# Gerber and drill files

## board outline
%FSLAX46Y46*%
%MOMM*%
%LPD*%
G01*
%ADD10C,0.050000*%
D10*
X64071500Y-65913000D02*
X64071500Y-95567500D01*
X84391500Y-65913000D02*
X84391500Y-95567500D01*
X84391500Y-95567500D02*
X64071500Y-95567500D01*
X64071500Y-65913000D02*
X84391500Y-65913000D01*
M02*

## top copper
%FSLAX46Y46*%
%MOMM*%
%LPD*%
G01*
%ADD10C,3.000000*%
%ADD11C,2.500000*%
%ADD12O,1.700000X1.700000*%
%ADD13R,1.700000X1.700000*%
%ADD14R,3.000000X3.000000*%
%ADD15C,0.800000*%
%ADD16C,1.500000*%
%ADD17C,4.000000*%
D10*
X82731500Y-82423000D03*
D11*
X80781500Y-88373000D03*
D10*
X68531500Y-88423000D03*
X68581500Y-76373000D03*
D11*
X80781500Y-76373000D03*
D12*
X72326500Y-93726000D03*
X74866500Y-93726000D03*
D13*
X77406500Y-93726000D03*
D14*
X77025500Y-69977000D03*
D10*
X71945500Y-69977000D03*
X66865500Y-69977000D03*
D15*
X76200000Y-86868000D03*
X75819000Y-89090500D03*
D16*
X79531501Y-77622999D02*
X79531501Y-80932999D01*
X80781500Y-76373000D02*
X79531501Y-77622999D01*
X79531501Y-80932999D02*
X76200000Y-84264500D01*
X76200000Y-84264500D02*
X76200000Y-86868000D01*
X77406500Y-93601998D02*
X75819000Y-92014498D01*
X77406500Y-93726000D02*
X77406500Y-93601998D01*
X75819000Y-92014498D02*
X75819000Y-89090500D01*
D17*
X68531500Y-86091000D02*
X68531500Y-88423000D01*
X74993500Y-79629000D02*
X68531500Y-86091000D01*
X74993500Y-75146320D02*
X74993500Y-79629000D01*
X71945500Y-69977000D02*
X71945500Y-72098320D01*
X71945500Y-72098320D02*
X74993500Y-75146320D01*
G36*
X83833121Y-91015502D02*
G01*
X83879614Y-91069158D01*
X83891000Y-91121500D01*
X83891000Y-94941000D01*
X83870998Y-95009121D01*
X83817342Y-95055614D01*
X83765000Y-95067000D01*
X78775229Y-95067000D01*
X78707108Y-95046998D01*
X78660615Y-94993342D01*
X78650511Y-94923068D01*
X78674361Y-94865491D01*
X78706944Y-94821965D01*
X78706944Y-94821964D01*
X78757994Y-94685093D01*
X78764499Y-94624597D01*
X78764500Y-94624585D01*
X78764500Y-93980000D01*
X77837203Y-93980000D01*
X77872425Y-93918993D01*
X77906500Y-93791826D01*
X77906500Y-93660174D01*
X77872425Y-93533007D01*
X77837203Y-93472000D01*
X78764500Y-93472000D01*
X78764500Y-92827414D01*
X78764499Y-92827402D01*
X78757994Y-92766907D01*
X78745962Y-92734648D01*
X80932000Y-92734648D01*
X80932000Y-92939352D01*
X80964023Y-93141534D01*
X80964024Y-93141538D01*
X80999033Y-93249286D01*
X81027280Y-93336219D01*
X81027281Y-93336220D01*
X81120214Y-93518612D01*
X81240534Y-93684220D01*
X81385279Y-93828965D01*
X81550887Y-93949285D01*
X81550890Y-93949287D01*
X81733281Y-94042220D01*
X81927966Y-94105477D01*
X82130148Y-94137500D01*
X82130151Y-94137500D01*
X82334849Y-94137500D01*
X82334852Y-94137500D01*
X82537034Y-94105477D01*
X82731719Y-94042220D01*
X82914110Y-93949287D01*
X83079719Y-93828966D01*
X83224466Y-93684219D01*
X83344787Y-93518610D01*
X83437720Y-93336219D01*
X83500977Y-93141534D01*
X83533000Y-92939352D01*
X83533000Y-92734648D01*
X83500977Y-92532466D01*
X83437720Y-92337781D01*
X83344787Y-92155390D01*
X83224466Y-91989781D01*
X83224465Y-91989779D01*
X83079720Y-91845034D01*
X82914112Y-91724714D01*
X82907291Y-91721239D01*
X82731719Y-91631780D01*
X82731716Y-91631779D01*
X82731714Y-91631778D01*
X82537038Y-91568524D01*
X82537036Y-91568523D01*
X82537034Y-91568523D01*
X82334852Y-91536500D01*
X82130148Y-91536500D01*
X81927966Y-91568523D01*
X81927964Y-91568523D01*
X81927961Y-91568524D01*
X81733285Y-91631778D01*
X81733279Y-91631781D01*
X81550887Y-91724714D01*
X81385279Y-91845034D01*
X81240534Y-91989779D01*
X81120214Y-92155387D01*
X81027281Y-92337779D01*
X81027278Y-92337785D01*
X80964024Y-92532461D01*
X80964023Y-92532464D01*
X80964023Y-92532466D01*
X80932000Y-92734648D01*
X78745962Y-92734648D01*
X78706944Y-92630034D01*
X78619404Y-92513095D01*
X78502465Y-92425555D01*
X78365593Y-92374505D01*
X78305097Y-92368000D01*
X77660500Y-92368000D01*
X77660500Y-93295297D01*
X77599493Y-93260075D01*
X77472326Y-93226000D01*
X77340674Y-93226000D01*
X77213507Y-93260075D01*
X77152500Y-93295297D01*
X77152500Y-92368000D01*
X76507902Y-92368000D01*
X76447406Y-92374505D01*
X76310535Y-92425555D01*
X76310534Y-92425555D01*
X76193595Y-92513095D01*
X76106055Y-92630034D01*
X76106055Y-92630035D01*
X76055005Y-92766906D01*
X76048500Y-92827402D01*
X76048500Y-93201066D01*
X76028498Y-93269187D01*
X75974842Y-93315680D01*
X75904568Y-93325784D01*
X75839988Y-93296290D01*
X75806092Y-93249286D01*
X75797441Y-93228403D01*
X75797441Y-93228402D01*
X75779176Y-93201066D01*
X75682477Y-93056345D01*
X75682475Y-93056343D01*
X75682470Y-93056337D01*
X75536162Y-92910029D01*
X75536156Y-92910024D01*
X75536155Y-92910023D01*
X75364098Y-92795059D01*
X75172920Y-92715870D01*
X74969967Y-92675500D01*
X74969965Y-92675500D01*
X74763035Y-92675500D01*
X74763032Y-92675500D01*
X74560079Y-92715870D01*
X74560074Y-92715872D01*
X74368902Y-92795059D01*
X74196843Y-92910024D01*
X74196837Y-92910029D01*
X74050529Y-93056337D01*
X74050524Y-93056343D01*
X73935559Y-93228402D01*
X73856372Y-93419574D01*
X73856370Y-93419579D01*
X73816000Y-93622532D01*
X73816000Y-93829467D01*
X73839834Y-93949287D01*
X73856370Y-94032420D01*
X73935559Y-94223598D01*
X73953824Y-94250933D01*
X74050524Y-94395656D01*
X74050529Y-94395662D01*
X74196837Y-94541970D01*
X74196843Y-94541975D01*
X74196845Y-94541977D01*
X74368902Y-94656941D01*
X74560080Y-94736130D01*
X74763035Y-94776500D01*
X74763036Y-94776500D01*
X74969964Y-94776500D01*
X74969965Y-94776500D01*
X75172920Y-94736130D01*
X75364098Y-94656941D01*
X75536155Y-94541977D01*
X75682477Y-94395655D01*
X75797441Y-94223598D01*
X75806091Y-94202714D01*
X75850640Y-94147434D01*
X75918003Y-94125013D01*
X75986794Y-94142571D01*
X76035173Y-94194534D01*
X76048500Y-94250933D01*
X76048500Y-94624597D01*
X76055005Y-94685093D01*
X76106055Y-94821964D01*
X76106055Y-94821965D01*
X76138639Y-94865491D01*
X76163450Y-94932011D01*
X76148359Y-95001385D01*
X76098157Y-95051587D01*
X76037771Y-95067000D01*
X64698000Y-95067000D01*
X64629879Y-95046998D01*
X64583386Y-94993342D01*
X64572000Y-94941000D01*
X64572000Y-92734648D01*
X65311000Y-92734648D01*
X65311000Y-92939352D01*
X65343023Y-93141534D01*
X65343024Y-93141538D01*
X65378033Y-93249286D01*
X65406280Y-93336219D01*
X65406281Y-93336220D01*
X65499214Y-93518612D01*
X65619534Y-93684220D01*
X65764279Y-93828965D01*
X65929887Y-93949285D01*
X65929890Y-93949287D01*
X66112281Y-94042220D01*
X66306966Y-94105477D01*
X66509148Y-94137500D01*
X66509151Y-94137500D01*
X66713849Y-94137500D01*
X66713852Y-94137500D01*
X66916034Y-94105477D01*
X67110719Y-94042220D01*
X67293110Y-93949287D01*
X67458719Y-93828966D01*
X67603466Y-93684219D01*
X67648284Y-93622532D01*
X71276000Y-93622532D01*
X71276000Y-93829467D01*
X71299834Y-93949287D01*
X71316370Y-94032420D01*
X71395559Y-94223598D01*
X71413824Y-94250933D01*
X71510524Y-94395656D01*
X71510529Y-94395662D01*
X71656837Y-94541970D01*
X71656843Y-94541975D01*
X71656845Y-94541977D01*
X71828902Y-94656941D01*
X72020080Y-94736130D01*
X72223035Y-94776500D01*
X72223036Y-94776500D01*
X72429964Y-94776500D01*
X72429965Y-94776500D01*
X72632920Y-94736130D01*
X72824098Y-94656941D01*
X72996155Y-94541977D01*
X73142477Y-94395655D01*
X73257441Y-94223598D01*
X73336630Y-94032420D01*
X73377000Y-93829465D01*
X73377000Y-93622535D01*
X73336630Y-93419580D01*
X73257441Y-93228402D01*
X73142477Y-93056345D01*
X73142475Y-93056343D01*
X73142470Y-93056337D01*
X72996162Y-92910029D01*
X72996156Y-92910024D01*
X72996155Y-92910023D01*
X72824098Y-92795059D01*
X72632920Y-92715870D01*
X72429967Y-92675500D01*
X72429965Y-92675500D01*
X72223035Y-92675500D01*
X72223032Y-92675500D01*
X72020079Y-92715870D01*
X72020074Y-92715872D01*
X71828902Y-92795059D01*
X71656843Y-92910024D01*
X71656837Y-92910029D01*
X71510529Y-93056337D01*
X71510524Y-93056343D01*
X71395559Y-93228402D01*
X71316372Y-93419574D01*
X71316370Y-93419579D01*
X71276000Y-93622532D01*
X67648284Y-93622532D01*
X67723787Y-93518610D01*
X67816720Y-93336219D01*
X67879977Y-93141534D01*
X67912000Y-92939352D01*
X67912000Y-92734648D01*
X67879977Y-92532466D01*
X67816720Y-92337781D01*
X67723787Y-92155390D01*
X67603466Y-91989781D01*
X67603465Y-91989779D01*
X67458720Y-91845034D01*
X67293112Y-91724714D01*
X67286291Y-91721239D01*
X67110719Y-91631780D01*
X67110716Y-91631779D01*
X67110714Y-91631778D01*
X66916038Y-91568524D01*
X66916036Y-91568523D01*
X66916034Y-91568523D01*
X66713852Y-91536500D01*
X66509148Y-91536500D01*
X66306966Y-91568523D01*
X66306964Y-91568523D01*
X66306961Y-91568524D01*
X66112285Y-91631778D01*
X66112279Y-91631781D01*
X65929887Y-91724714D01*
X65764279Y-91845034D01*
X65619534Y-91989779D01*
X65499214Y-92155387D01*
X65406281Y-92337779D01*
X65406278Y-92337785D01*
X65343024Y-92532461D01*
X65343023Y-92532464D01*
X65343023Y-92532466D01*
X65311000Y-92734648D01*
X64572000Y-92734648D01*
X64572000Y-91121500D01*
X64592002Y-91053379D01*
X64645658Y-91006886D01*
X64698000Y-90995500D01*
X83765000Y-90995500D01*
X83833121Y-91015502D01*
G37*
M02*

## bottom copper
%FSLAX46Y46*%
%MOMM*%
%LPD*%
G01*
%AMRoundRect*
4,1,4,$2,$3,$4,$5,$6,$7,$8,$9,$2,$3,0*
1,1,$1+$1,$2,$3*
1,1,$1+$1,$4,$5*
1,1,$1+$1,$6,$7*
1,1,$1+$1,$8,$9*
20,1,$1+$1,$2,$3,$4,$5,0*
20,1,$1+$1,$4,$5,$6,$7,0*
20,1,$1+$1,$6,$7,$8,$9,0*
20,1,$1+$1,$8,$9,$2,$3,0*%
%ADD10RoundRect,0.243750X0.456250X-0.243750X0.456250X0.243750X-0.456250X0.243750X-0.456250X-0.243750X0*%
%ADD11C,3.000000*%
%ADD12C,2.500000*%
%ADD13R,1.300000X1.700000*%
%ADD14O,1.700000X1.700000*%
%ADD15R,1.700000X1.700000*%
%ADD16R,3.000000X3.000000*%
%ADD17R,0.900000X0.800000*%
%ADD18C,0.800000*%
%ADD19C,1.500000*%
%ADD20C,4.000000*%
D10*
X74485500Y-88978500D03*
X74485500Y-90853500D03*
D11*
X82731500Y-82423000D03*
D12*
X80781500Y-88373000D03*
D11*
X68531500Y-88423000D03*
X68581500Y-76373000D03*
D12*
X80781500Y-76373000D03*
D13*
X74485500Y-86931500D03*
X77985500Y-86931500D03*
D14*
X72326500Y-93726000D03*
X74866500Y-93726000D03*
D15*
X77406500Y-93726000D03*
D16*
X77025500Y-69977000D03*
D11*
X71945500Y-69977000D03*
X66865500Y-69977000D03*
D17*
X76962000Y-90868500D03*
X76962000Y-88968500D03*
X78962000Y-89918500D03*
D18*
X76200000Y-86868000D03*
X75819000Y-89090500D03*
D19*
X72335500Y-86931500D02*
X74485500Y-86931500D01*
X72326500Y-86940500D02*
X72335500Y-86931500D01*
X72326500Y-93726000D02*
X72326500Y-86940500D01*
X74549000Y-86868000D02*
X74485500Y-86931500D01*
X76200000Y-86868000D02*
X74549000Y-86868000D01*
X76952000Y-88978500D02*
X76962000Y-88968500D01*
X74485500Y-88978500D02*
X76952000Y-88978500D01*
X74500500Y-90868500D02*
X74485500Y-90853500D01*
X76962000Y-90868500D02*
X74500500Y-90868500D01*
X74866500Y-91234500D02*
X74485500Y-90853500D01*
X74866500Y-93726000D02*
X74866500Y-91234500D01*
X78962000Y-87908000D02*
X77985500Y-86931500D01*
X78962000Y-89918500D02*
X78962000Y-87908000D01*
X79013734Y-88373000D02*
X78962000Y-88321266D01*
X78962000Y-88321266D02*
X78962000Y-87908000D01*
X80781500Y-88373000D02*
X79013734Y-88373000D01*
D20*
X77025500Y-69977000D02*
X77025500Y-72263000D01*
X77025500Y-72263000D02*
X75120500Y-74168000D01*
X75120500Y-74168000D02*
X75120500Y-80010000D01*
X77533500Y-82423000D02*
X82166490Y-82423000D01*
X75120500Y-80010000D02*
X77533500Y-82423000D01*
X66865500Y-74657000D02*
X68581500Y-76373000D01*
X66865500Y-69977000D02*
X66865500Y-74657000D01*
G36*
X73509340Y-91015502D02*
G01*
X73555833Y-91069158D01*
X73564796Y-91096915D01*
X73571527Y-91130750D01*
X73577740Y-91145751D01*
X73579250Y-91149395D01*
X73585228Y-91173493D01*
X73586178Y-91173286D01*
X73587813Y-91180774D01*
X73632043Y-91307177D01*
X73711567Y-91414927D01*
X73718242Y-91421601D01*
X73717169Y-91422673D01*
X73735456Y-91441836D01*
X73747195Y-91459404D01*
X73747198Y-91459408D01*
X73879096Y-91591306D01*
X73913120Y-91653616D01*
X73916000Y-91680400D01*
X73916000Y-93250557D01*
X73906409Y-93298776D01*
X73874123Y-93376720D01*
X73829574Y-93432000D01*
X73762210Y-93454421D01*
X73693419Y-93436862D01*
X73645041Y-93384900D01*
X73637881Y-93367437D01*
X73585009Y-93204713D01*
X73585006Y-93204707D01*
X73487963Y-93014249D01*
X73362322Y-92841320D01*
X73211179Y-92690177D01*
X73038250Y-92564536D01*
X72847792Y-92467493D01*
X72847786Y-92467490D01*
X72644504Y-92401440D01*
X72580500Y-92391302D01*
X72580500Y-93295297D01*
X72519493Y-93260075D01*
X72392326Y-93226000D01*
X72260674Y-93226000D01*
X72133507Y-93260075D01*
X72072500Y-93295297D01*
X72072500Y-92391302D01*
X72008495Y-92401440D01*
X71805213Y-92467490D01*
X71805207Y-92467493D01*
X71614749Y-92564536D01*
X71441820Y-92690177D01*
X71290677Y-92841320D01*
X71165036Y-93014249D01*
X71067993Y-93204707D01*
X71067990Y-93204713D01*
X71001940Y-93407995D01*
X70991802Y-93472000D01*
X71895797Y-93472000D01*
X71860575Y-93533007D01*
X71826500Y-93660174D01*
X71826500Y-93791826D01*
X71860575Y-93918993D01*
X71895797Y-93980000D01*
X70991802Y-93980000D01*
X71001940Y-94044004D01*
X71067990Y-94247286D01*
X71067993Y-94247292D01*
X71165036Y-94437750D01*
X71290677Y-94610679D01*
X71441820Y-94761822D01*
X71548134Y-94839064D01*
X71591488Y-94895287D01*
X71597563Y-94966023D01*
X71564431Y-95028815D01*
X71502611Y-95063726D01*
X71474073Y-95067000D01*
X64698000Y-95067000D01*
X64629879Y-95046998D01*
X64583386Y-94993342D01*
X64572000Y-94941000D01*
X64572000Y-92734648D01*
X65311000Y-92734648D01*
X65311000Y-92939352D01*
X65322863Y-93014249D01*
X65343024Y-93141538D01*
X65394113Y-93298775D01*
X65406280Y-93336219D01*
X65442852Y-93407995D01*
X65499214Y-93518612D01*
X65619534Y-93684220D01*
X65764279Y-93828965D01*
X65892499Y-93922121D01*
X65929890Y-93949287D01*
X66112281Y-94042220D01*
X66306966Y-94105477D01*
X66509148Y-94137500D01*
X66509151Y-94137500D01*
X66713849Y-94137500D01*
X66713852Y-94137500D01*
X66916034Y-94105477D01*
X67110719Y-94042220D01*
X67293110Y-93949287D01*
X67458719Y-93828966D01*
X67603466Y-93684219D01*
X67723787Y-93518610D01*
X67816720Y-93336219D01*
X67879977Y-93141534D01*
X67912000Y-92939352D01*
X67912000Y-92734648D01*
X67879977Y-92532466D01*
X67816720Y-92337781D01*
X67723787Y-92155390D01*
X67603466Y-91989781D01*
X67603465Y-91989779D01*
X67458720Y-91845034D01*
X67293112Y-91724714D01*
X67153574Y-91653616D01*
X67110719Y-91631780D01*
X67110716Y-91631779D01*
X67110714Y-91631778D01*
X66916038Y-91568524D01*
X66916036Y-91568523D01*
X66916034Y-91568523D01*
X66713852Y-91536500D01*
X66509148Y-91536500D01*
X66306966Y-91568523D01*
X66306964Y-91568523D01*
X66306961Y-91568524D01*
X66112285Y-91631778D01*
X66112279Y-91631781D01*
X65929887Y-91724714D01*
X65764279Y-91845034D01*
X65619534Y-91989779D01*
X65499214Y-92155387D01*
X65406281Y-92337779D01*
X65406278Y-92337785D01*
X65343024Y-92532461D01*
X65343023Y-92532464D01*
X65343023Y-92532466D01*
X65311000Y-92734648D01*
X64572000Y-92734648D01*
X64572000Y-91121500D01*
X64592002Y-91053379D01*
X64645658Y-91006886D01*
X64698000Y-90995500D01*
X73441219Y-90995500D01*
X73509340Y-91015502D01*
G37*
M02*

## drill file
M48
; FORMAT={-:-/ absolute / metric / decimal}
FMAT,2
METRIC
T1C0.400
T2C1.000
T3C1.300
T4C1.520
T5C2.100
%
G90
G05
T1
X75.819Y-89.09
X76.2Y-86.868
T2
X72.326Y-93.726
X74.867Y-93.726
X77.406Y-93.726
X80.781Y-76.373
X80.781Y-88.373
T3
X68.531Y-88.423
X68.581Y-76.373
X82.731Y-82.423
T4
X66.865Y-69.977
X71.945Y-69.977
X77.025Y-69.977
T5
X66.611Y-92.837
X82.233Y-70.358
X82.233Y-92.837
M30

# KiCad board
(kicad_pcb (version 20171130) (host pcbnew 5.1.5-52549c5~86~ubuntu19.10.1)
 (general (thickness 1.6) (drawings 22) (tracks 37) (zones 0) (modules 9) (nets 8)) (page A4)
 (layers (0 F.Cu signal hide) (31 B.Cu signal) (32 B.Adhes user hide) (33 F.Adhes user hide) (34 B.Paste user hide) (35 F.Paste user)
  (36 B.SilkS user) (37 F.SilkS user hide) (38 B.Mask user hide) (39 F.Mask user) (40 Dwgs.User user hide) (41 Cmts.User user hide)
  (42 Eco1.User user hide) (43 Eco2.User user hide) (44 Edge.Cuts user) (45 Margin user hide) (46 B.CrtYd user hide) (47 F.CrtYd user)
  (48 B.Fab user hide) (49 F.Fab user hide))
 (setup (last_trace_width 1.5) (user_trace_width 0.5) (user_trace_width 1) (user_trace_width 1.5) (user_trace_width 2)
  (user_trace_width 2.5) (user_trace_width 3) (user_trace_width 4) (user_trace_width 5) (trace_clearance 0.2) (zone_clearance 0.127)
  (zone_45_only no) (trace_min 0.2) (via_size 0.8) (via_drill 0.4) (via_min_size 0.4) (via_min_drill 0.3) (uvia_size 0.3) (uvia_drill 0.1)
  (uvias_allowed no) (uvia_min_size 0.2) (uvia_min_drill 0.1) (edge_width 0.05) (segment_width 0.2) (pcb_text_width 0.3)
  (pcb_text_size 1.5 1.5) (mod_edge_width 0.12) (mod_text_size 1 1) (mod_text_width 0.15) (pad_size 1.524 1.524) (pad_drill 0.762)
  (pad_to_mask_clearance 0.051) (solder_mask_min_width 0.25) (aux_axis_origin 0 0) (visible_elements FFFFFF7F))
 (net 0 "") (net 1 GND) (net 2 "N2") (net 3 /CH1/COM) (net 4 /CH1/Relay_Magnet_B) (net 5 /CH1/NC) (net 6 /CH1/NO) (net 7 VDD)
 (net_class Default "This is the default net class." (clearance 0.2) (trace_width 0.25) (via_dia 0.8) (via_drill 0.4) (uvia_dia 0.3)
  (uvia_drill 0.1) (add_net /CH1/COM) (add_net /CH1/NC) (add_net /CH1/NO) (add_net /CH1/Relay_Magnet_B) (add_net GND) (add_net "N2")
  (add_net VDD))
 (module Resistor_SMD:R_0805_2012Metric (layer B.Cu) (at 74.4855 89.916 90)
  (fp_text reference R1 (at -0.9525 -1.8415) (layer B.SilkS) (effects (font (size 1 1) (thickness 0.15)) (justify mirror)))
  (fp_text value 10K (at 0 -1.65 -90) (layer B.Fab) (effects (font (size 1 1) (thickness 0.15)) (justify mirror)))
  (pad 2 smd roundrect (at 0.9375 0 90) (size 0.975 1.4) (layers B.Cu B.Paste B.Mask) (roundrect_rratio 0.25) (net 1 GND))
  (pad 1 smd roundrect (at -0.9375 0 90) (size 0.975 1.4) (layers B.Cu B.Paste B.Mask) (roundrect_rratio 0.25) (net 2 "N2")))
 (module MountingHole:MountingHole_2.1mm (layer F.Cu) (at 66.6115 92.837)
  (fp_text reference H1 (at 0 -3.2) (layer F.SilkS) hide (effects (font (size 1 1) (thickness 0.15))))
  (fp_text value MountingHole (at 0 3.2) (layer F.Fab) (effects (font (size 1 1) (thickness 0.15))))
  (pad "" np_thru_hole circle (at 0 0) (size 2.1 2.1) (drill 2.1) (layers *.Cu *.Mask)))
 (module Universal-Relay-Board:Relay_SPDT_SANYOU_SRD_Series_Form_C (layer F.Cu) (at 82.7315 82.423 180)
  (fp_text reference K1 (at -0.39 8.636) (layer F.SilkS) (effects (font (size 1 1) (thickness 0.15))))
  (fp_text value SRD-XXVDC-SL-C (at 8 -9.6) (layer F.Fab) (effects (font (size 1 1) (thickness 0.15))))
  (pad 1 thru_hole circle (at 0 0 270) (size 3 3) (drill 1.3) (layers *.Cu *.Mask) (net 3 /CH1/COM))
  (pad 5 thru_hole circle (at 1.95 -5.95 270) (size 2.5 2.5) (drill 1) (layers *.Cu *.Mask) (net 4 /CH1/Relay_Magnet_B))
  (pad 4 thru_hole circle (at 14.2 -6 270) (size 3 3) (drill 1.3) (layers *.Cu *.Mask) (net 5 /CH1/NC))
  (pad 3 thru_hole circle (at 14.15 6.05 270) (size 3 3) (drill 1.3) (layers *.Cu *.Mask) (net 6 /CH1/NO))
  (pad 2 thru_hole circle (at 1.95 6.05 270) (size 2.5 2.5) (drill 1) (layers *.Cu *.Mask) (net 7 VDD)))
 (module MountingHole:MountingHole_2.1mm (layer F.Cu) (at 82.2325 70.358)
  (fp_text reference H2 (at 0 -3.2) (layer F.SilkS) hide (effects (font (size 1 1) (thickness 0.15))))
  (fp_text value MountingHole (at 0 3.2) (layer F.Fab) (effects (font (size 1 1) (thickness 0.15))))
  (pad "" np_thru_hole circle (at 0 0) (size 2.1 2.1) (drill 2.1) (layers *.Cu *.Mask)))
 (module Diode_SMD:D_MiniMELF (layer B.Cu) (at 76.2355 86.9315)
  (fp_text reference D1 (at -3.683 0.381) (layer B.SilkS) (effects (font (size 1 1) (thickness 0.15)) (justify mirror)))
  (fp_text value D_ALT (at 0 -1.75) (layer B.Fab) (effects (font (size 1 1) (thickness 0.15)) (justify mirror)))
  (pad 1 smd rect (at -1.75 0) (size 1.3 1.7) (layers B.Cu B.Paste B.Mask) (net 7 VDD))
  (pad 2 smd rect (at 1.75 0) (size 1.3 1.7) (layers B.Cu B.Paste B.Mask) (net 4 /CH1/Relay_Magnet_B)))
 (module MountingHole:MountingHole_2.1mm (layer F.Cu) (at 82.2325 92.837)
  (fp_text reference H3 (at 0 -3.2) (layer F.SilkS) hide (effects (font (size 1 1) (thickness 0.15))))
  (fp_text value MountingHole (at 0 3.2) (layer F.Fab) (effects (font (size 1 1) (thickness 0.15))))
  (pad "" np_thru_hole circle (at 0 0) (size 2.1 2.1) (drill 2.1) (layers *.Cu *.Mask)))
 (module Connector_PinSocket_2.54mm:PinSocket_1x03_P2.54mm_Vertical (layer F.Cu) (at 77.4065 93.726 270)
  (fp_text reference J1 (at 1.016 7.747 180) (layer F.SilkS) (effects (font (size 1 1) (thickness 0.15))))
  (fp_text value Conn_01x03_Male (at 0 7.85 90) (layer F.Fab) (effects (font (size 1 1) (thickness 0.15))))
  (pad 3 thru_hole oval (at 0 5.08 270) (size 1.7 1.7) (drill 1) (layers *.Cu *.Mask) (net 7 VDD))
  (pad 2 thru_hole oval (at 0 2.54 270) (size 1.7 1.7) (drill 1) (layers *.Cu *.Mask) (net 2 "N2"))
  (pad 1 thru_hole rect (at 0 0 270) (size 1.7 1.7) (drill 1) (layers *.Cu *.Mask) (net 1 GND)))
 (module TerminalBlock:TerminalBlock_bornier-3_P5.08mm (layer F.Cu) (at 77.0255 69.977 180)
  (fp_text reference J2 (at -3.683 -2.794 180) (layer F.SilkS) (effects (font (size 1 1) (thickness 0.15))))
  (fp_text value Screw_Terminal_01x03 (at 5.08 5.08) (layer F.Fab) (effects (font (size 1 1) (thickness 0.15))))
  (pad 1 thru_hole rect (at 0 0 180) (size 3 3) (drill 1.52) (layers *.Cu *.Mask) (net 3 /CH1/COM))
  (pad 2 thru_hole circle (at 5.08 0 180) (size 3 3) (drill 1.52) (layers *.Cu *.Mask) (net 5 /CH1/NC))
  (pad 3 thru_hole circle (at 10.16 0 180) (size 3 3) (drill 1.52) (layers *.Cu *.Mask) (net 6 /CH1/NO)))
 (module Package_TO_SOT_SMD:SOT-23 (layer B.Cu) (at 77.962 89.9185)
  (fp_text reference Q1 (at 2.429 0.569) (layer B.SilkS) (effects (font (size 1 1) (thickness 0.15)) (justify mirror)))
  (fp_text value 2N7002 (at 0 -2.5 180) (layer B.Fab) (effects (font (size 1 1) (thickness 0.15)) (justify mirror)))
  (pad 1 smd rect (at -1 0.95) (size 0.9 0.8) (layers B.Cu B.Paste B.Mask) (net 2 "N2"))
  (pad 2 smd rect (at -1 -0.95) (size 0.9 0.8) (layers B.Cu B.Paste B.Mask) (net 1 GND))
  (pad 3 smd rect (at 1 0) (size 0.9 0.8) (layers B.Cu B.Paste B.Mask) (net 4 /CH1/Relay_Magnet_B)))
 (gr_line (start 64.0715 65.913) (end 64.0715 95.5675) (layer Edge.Cuts) (width 0.05))
 (gr_line (start 84.3915 65.913) (end 84.3915 95.5675) (layer Edge.Cuts) (width 0.05))
 (gr_line (start 84.3915 95.5675) (end 64.0715 95.5675) (layer Edge.Cuts) (width 0.05))
 (gr_line (start 64.0715 65.913) (end 84.3915 65.913) (layer Edge.Cuts) (width 0.05))
 (segment (start 72.3355 86.9315) (end 74.4855 86.9315) (width 1.5) (layer B.Cu) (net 7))
 (segment (start 72.3265 86.9405) (end 72.3355 86.9315) (width 1.5) (layer B.Cu) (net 7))
 (segment (start 72.3265 93.726) (end 72.3265 86.9405) (width 1.5) (layer B.Cu) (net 7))
 (segment (start 79.531501 77.622999) (end 79.531501 80.932999) (width 1.5) (layer F.Cu) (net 7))
 (segment (start 80.7815 76.373) (end 79.531501 77.622999) (width 1.5) (layer F.Cu) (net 7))
 (segment (start 79.531501 80.932999) (end 76.2 84.2645) (width 1.5) (layer F.Cu) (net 7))
 (segment (start 76.2 84.2645) (end 76.2 86.868) (width 1.5) (layer F.Cu) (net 7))
 (via (at 76.2 86.868) (size 0.8) (drill 0.4) (layers F.Cu B.Cu) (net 7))
 (segment (start 74.549 86.868) (end 74.4855 86.9315) (width 1.5) (layer B.Cu) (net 7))
 (segment (start 76.2 86.868) (end 74.549 86.868) (width 1.5) (layer B.Cu) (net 7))
 (segment (start 76.952 88.9785) (end 76.962 88.9685) (width 1.5) (layer B.Cu) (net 1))
 (segment (start 74.4855 88.9785) (end 76.952 88.9785) (width 1.5) (layer B.Cu) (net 1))
 (segment (start 77.4065 93.601998) (end 75.819 92.014498) (width 1.5) (layer F.Cu) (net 1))
 (segment (start 77.4065 93.726) (end 77.4065 93.601998) (width 1.5) (layer F.Cu) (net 1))
 (segment (start 75.819 92.014498) (end 75.819 89.0905) (width 1.5) (layer F.Cu) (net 1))
 (via (at 75.819 89.0905) (size 0.8) (drill 0.4) (layers F.Cu B.Cu) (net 1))
 (segment (start 74.5005 90.8685) (end 74.4855 90.8535) (width 1.5) (layer B.Cu) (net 2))
 (segment (start 76.962 90.8685) (end 74.5005 90.8685) (width 1.5) (layer B.Cu) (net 2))
 (segment (start 74.8665 91.2345) (end 74.4855 90.8535) (width 1.5) (layer B.Cu) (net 2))
 (segment (start 74.8665 93.726) (end 74.8665 91.2345) (width 1.5) (layer B.Cu) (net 2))
 (segment (start 78.962 87.908) (end 77.9855 86.9315) (width 1.5) (layer B.Cu) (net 4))
 (segment (start 78.962 89.9185) (end 78.962 87.908) (width 1.5) (layer B.Cu) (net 4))
 (segment (start 79.013734 88.373) (end 78.962 88.321266) (width 1.5) (layer B.Cu) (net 4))
 (segment (start 78.962 88.321266) (end 78.962 87.908) (width 1.5) (layer B.Cu) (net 4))
 (segment (start 80.7815 88.373) (end 79.013734 88.373) (width 1.5) (layer B.Cu) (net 4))
 (segment (start 77.0255 69.977) (end 77.0255 72.263) (width 4) (layer B.Cu) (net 3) (status 10))
 (segment (start 77.0255 72.263) (end 75.1205 74.168) (width 4) (layer B.Cu) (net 3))
 (segment (start 75.1205 74.168) (end 75.1205 80.01) (width 4) (layer B.Cu) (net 3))
 (segment (start 77.5335 82.423) (end 82.16649 82.423) (width 4) (layer B.Cu) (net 3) (status 20))
 (segment (start 75.1205 80.01) (end 77.5335 82.423) (width 4) (layer B.Cu) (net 3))
 (segment (start 66.8655 74.657) (end 68.5815 76.373) (width 4) (layer B.Cu) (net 6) (status 20))
 (segment (start 66.8655 69.977) (end 66.8655 74.657) (width 4) (layer B.Cu) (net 6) (status 10))
 (segment (start 68.5315 86.091) (end 68.5315 88.423) (width 4) (layer F.Cu) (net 5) (status 20))
 (segment (start 74.9935 79.629) (end 68.5315 86.091) (width 4) (layer F.Cu) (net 5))
 (segment (start 74.9935 75.14632) (end 74.9935 79.629) (width 4) (layer F.Cu) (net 5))
 (segment (start 71.9455 69.977) (end 71.9455 72.09832) (width 4) (layer F.Cu) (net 5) (status 10))
 (segment (start 71.9455 72.09832) (end 74.9935 75.14632) (width 4) (layer F.Cu) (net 5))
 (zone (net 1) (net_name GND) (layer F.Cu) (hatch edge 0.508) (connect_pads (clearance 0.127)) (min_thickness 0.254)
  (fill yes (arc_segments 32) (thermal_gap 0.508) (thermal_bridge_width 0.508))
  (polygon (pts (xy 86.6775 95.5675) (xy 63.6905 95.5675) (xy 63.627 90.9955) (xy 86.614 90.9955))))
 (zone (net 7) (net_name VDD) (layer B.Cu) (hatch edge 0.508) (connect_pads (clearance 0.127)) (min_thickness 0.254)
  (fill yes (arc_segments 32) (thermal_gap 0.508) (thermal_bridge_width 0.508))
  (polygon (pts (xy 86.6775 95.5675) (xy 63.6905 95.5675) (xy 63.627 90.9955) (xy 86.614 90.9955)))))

